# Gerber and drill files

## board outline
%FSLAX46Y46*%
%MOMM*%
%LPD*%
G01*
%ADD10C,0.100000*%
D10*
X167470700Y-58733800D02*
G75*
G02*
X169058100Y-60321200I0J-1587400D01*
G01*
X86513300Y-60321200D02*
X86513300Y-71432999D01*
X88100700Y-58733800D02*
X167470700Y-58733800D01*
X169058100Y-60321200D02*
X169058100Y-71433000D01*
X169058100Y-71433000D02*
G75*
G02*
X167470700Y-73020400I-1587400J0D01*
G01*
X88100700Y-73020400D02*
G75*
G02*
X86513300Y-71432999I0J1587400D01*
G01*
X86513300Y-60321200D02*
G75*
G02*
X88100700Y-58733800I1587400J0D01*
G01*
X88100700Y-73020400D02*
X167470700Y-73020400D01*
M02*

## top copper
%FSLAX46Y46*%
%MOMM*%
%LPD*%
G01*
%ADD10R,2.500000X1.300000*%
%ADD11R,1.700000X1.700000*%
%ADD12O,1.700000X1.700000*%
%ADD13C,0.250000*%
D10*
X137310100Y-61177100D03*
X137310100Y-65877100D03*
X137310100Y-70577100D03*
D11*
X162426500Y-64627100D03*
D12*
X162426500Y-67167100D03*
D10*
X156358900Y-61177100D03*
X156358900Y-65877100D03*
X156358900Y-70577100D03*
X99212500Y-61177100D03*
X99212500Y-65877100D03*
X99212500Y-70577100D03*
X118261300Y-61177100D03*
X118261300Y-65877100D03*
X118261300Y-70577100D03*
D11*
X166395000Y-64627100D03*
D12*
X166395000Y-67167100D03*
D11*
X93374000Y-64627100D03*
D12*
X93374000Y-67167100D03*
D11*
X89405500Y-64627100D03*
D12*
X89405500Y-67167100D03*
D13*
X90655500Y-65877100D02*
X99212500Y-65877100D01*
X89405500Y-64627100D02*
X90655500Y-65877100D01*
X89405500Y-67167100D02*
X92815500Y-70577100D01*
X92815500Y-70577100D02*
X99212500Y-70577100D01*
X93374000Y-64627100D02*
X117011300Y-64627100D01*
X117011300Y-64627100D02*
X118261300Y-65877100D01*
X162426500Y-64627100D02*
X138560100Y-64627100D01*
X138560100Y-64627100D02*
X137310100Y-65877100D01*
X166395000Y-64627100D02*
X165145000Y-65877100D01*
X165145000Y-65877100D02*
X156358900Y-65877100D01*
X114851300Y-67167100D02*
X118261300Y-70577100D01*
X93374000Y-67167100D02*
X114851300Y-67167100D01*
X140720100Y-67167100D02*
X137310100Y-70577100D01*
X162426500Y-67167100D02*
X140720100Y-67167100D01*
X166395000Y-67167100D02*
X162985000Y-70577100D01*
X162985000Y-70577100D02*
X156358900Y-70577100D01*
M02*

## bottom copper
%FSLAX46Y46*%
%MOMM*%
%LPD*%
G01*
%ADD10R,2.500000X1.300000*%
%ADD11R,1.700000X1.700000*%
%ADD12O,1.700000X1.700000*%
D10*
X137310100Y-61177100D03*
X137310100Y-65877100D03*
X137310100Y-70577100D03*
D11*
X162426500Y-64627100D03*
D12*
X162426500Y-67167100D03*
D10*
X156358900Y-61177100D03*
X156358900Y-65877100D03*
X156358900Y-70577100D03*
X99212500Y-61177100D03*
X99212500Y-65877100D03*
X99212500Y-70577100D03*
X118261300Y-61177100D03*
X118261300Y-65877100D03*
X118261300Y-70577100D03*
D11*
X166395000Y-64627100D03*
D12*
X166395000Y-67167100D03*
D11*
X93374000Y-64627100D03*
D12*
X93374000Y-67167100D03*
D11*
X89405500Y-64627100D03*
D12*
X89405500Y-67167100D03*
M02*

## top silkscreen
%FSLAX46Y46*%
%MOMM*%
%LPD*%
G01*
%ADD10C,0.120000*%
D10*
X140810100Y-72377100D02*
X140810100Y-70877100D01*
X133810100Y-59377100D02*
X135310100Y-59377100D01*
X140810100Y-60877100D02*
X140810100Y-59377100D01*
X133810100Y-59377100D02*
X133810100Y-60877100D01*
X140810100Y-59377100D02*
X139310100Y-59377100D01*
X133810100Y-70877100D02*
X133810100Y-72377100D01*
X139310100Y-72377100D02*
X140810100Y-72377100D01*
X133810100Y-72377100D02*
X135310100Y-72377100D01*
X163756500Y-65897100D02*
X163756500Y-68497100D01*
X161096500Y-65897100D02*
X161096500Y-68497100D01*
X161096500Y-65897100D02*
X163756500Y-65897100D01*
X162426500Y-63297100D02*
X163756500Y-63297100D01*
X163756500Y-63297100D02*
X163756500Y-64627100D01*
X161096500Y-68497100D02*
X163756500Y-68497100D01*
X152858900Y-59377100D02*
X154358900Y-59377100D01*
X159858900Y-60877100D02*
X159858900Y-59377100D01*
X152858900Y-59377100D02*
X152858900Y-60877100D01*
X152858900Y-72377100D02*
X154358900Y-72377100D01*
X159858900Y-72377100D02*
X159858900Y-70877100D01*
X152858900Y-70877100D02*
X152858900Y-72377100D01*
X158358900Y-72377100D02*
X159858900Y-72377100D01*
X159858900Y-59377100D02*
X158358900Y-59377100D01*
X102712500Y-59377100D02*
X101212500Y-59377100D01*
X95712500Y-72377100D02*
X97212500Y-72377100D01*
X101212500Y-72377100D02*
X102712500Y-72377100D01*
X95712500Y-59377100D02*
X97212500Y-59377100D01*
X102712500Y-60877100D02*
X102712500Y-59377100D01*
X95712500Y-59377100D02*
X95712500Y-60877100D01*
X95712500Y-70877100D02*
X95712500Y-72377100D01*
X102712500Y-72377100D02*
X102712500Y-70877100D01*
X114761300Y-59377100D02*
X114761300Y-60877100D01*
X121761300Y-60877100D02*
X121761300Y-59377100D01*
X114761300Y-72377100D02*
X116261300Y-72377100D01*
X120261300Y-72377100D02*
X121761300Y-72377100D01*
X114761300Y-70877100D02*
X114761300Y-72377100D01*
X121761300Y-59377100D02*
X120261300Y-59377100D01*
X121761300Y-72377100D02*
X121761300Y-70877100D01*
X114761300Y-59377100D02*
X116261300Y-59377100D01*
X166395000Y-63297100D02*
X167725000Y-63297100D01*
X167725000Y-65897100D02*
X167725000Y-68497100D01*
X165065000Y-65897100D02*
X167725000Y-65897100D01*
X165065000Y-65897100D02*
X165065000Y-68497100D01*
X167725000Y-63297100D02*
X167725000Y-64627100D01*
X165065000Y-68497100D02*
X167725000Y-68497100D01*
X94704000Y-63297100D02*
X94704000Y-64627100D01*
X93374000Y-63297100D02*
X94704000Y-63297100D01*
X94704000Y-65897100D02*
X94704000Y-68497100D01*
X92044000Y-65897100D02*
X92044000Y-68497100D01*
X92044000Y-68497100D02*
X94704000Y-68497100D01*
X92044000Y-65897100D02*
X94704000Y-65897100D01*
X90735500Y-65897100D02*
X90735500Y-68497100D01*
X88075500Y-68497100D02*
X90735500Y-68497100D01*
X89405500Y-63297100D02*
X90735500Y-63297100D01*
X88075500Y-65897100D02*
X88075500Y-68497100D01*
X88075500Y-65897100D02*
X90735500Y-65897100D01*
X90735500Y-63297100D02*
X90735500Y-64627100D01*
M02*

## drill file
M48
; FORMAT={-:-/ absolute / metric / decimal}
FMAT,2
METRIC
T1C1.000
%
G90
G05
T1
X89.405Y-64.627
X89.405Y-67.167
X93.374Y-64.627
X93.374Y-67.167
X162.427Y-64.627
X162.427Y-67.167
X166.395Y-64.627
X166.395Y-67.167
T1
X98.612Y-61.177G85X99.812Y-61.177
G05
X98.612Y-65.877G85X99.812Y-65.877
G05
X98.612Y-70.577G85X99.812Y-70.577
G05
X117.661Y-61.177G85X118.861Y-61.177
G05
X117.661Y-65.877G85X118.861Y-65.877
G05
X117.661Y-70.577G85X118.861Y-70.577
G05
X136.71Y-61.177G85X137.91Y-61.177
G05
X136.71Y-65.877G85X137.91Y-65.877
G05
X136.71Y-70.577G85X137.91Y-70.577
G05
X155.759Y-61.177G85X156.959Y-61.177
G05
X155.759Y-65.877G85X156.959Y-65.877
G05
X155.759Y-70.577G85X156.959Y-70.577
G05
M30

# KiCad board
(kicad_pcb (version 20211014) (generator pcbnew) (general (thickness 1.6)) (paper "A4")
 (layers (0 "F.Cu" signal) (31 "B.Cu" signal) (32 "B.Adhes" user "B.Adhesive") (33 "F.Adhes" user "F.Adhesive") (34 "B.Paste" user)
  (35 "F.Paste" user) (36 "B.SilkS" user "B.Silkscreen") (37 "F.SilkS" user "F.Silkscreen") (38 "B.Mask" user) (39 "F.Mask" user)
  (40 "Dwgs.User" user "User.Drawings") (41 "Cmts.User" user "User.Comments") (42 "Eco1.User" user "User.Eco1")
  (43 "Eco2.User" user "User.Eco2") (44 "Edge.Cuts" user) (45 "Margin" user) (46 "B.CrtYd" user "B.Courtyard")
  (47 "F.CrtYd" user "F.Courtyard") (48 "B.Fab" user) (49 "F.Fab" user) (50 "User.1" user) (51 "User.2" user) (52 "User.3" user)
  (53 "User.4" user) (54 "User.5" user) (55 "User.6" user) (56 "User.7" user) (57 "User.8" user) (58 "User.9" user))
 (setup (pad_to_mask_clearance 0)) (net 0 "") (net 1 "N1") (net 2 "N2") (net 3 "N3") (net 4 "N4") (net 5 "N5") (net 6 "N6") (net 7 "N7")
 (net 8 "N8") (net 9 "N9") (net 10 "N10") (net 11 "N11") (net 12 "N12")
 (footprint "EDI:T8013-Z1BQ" (layer "F.Cu") (at 137.3101 65.8771)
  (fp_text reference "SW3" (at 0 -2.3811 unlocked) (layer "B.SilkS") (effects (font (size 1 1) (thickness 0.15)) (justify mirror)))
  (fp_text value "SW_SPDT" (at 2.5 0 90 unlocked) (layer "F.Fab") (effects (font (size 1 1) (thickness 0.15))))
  (fp_line (start 3.5 6.5) (end 3.5 5) (layer "F.SilkS") (width 0.12))
  (fp_line (start -3.5 -6.5) (end -2 -6.5) (layer "F.SilkS") (width 0.12))
  (fp_line (start 3.5 -5) (end 3.5 -6.5) (layer "F.SilkS") (width 0.12))
  (fp_line (start -3.5 -6.5) (end -3.5 -5) (layer "F.SilkS") (width 0.12))
  (fp_line (start 3.5 -6.5) (end 2 -6.5) (layer "F.SilkS") (width 0.12))
  (fp_line (start -3.5 5) (end -3.5 6.5) (layer "F.SilkS") (width 0.12))
  (fp_line (start 2 6.5) (end 3.5 6.5) (layer "F.SilkS") (width 0.12))
  (fp_line (start -3.5 6.5) (end -2 6.5) (layer "F.SilkS") (width 0.12))
  (pad "1" thru_hole rect (at 0 -4.7) (size 2.5 1.3) (drill oval 2.2 1) (layers *.Cu *.Mask) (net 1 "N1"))
  (pad "2" thru_hole rect (at 0 0) (size 2.5 1.3) (drill oval 2.2 1) (layers *.Cu *.Mask) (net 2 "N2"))
  (pad "3" thru_hole rect (at 0 4.7) (size 2.5 1.3) (drill oval 2.2 1) (layers *.Cu *.Mask) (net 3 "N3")))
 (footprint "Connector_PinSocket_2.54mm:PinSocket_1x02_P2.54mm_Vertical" (layer "F.Cu") (at 162.4265 64.6271)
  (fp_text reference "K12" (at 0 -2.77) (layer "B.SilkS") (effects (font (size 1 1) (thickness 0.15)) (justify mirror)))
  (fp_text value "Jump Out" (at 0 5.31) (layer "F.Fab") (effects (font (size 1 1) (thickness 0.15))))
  (fp_line (start 1.33 1.27) (end 1.33 3.87) (layer "F.SilkS") (width 0.12))
  (fp_line (start -1.33 1.27) (end -1.33 3.87) (layer "F.SilkS") (width 0.12))
  (fp_line (start -1.33 1.27) (end 1.33 1.27) (layer "F.SilkS") (width 0.12))
  (fp_line (start 0 -1.33) (end 1.33 -1.33) (layer "F.SilkS") (width 0.12))
  (fp_line (start 1.33 -1.33) (end 1.33 0) (layer "F.SilkS") (width 0.12))
  (fp_line (start -1.33 3.87) (end 1.33 3.87) (layer "F.SilkS") (width 0.12))
  (pad "1" thru_hole rect locked (at 0 0) (size 1.7 1.7) (drill 1) (layers *.Cu *.Mask) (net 2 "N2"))
  (pad "2" thru_hole oval locked (at 0 2.54) (size 1.7 1.7) (drill 1) (layers *.Cu *.Mask) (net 3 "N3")))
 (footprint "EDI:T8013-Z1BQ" (layer "F.Cu") (at 156.3589 65.8771)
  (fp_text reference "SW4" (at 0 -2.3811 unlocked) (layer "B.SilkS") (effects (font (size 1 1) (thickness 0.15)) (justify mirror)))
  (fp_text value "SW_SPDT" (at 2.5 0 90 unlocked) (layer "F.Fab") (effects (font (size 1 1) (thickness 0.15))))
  (fp_line (start -3.5 -6.5) (end -2 -6.5) (layer "F.SilkS") (width 0.12))
  (fp_line (start 3.5 -5) (end 3.5 -6.5) (layer "F.SilkS") (width 0.12))
  (fp_line (start -3.5 -6.5) (end -3.5 -5) (layer "F.SilkS") (width 0.12))
  (fp_line (start -3.5 6.5) (end -2 6.5) (layer "F.SilkS") (width 0.12))
  (fp_line (start 3.5 6.5) (end 3.5 5) (layer "F.SilkS") (width 0.12))
  (fp_line (start -3.5 5) (end -3.5 6.5) (layer "F.SilkS") (width 0.12))
  (fp_line (start 2 6.5) (end 3.5 6.5) (layer "F.SilkS") (width 0.12))
  (fp_line (start 3.5 -6.5) (end 2 -6.5) (layer "F.SilkS") (width 0.12))
  (pad "1" thru_hole rect (at 0 -4.7) (size 2.5 1.3) (drill oval 2.2 1) (layers *.Cu *.Mask) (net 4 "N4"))
  (pad "2" thru_hole rect (at 0 0) (size 2.5 1.3) (drill oval 2.2 1) (layers *.Cu *.Mask) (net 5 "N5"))
  (pad "3" thru_hole rect (at 0 4.7) (size 2.5 1.3) (drill oval 2.2 1) (layers *.Cu *.Mask) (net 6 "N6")))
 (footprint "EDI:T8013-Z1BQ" (layer "F.Cu") (at 99.2125 65.8771)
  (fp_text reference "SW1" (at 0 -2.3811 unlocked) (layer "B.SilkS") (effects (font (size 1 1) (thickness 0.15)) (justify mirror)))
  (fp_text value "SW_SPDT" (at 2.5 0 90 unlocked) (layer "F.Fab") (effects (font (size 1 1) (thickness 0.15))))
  (fp_line (start 3.5 -6.5) (end 2 -6.5) (layer "F.SilkS") (width 0.12))
  (fp_line (start -3.5 6.5) (end -2 6.5) (layer "F.SilkS") (width 0.12))
  (fp_line (start 2 6.5) (end 3.5 6.5) (layer "F.SilkS") (width 0.12))
  (fp_line (start -3.5 -6.5) (end -2 -6.5) (layer "F.SilkS") (width 0.12))
  (fp_line (start 3.5 -5) (end 3.5 -6.5) (layer "F.SilkS") (width 0.12))
  (fp_line (start -3.5 -6.5) (end -3.5 -5) (layer "F.SilkS") (width 0.12))
  (fp_line (start -3.5 5) (end -3.5 6.5) (layer "F.SilkS") (width 0.12))
  (fp_line (start 3.5 6.5) (end 3.5 5) (layer "F.SilkS") (width 0.12))
  (pad "1" thru_hole rect (at 0 -4.7) (size 2.5 1.3) (drill oval 2.2 1) (layers *.Cu *.Mask) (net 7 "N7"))
  (pad "2" thru_hole rect (at 0 0) (size 2.5 1.3) (drill oval 2.2 1) (layers *.Cu *.Mask) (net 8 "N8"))
  (pad "3" thru_hole rect (at 0 4.7) (size 2.5 1.3) (drill oval 2.2 1) (layers *.Cu *.Mask) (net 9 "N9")))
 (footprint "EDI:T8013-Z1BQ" (layer "F.Cu") (at 118.2613 65.8771)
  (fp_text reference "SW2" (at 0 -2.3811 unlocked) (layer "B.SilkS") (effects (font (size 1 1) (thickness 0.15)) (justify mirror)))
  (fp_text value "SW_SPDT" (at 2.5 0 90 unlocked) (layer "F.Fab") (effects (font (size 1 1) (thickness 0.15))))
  (fp_line (start -3.5 -6.5) (end -3.5 -5) (layer "F.SilkS") (width 0.12))
  (fp_line (start 3.5 -5) (end 3.5 -6.5) (layer "F.SilkS") (width 0.12))
  (fp_line (start -3.5 6.5) (end -2 6.5) (layer "F.SilkS") (width 0.12))
  (fp_line (start 2 6.5) (end 3.5 6.5) (layer "F.SilkS") (width 0.12))
  (fp_line (start -3.5 5) (end -3.5 6.5) (layer "F.SilkS") (width 0.12))
  (fp_line (start 3.5 -6.5) (end 2 -6.5) (layer "F.SilkS") (width 0.12))
  (fp_line (start 3.5 6.5) (end 3.5 5) (layer "F.SilkS") (width 0.12))
  (fp_line (start -3.5 -6.5) (end -2 -6.5) (layer "F.SilkS") (width 0.12))
  (pad "1" thru_hole rect (at 0 -4.7) (size 2.5 1.3) (drill oval 2.2 1) (layers *.Cu *.Mask) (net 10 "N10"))
  (pad "2" thru_hole rect (at 0 0) (size 2.5 1.3) (drill oval 2.2 1) (layers *.Cu *.Mask) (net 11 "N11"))
  (pad "3" thru_hole rect (at 0 4.7) (size 2.5 1.3) (drill oval 2.2 1) (layers *.Cu *.Mask) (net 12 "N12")))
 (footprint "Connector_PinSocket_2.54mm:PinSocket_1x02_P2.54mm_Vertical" (layer "F.Cu") (at 166.395 64.6271)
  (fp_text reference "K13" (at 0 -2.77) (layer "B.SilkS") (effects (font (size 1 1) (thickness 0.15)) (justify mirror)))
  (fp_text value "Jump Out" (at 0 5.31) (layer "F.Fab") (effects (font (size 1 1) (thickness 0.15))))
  (fp_line (start 0 -1.33) (end 1.33 -1.33) (layer "F.SilkS") (width 0.12))
  (fp_line (start 1.33 1.27) (end 1.33 3.87) (layer "F.SilkS") (width 0.12))
  (fp_line (start -1.33 1.27) (end 1.33 1.27) (layer "F.SilkS") (width 0.12))
  (fp_line (start -1.33 1.27) (end -1.33 3.87) (layer "F.SilkS") (width 0.12))
  (fp_line (start 1.33 -1.33) (end 1.33 0) (layer "F.SilkS") (width 0.12))
  (fp_line (start -1.33 3.87) (end 1.33 3.87) (layer "F.SilkS") (width 0.12))
  (pad "1" thru_hole rect locked (at 0 0) (size 1.7 1.7) (drill 1) (layers *.Cu *.Mask) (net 5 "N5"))
  (pad "2" thru_hole oval locked (at 0 2.54) (size 1.7 1.7) (drill 1) (layers *.Cu *.Mask) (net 6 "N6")))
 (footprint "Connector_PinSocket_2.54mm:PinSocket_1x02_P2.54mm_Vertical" (layer "F.Cu") (at 93.374 64.6271)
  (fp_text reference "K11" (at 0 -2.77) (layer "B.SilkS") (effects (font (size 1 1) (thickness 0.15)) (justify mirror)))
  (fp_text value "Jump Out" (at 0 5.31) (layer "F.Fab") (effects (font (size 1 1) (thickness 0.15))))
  (fp_line (start 1.33 -1.33) (end 1.33 0) (layer "F.SilkS") (width 0.12))
  (fp_line (start 0 -1.33) (end 1.33 -1.33) (layer "F.SilkS") (width 0.12))
  (fp_line (start 1.33 1.27) (end 1.33 3.87) (layer "F.SilkS") (width 0.12))
  (fp_line (start -1.33 1.27) (end -1.33 3.87) (layer "F.SilkS") (width 0.12))
  (fp_line (start -1.33 3.87) (end 1.33 3.87) (layer "F.SilkS") (width 0.12))
  (fp_line (start -1.33 1.27) (end 1.33 1.27) (layer "F.SilkS") (width 0.12))
  (pad "1" thru_hole rect locked (at 0 0) (size 1.7 1.7) (drill 1) (layers *.Cu *.Mask) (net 11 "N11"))
  (pad "2" thru_hole oval locked (at 0 2.54) (size 1.7 1.7) (drill 1) (layers *.Cu *.Mask) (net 12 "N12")))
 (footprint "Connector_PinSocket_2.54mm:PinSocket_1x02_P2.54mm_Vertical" (layer "F.Cu") (at 89.4055 64.6271)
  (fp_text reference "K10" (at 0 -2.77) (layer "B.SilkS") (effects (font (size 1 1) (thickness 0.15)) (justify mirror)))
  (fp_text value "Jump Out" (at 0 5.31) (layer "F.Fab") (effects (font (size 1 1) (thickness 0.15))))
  (fp_line (start 1.33 1.27) (end 1.33 3.87) (layer "F.SilkS") (width 0.12))
  (fp_line (start -1.33 3.87) (end 1.33 3.87) (layer "F.SilkS") (width 0.12))
  (fp_line (start 0 -1.33) (end 1.33 -1.33) (layer "F.SilkS") (width 0.12))
  (fp_line (start -1.33 1.27) (end -1.33 3.87) (layer "F.SilkS") (width 0.12))
  (fp_line (start -1.33 1.27) (end 1.33 1.27) (layer "F.SilkS") (width 0.12))
  (fp_line (start 1.33 -1.33) (end 1.33 0) (layer "F.SilkS") (width 0.12))
  (pad "1" thru_hole rect locked (at 0 0) (size 1.7 1.7) (drill 1) (layers *.Cu *.Mask) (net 8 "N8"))
  (pad "2" thru_hole oval locked (at 0 2.54) (size 1.7 1.7) (drill 1) (layers *.Cu *.Mask) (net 9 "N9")))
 (gr_arc (start 167.4707 58.7338) (mid 168.593161 59.198739) (end 169.0581 60.3212) (layer "Edge.Cuts") (width 0.1))
 (gr_line (start 86.5133 60.3212) (end 86.5133 71.432999) (layer "Edge.Cuts") (width 0.1))
 (gr_line (start 88.1007 58.7338) (end 167.4707 58.7338) (layer "Edge.Cuts") (width 0.1))
 (gr_line (start 169.0581 60.3212) (end 169.0581 71.433) (layer "Edge.Cuts") (width 0.1))
 (gr_arc (start 169.0581 71.433) (mid 168.593161 72.555461) (end 167.4707 73.0204) (layer "Edge.Cuts") (width 0.1))
 (gr_arc (start 88.1007 73.0204) (mid 86.978239 72.555461) (end 86.5133 71.432999) (layer "Edge.Cuts") (width 0.1))
 (gr_arc (start 86.5133 60.3212) (mid 86.978239 59.198739) (end 88.1007 58.7338) (layer "Edge.Cuts") (width 0.1))
 (gr_line (start 88.1007 73.0204) (end 167.4707 73.0204) (layer "Edge.Cuts") (width 0.1))
 (segment (start 90.6555 65.8771) (end 99.2125 65.8771) (width 0.25) (layer "F.Cu") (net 8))
 (segment (start 89.4055 64.6271) (end 90.6555 65.8771) (width 0.25) (layer "F.Cu") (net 8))
 (segment (start 89.4055 67.1671) (end 92.8155 70.5771) (width 0.25) (layer "F.Cu") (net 9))
 (segment (start 92.8155 70.5771) (end 99.2125 70.5771) (width 0.25) (layer "F.Cu") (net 9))
 (segment (start 93.374 64.6271) (end 117.0113 64.6271) (width 0.25) (layer "F.Cu") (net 11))
 (segment (start 117.0113 64.6271) (end 118.2613 65.8771) (width 0.25) (layer "F.Cu") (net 11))
 (segment (start 162.4265 64.6271) (end 138.5601 64.6271) (width 0.25) (layer "F.Cu") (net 2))
 (segment (start 138.5601 64.6271) (end 137.3101 65.8771) (width 0.25) (layer "F.Cu") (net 2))
 (segment (start 166.395 64.6271) (end 165.145 65.8771) (width 0.25) (layer "F.Cu") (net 5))
 (segment (start 165.145 65.8771) (end 156.3589 65.8771) (width 0.25) (layer "F.Cu") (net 5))
 (segment (start 114.8513 67.1671) (end 118.2613 70.5771) (width 0.25) (layer "F.Cu") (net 12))
 (segment (start 93.374 67.1671) (end 114.8513 67.1671) (width 0.25) (layer "F.Cu") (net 12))
 (segment (start 140.7201 67.1671) (end 137.3101 70.5771) (width 0.25) (layer "F.Cu") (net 3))
 (segment (start 162.4265 67.1671) (end 140.7201 67.1671) (width 0.25) (layer "F.Cu") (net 3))
 (segment (start 166.395 67.1671) (end 162.985 70.5771) (width 0.25) (layer "F.Cu") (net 6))
 (segment (start 162.985 70.5771) (end 156.3589 70.5771) (width 0.25) (layer "F.Cu") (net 6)))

